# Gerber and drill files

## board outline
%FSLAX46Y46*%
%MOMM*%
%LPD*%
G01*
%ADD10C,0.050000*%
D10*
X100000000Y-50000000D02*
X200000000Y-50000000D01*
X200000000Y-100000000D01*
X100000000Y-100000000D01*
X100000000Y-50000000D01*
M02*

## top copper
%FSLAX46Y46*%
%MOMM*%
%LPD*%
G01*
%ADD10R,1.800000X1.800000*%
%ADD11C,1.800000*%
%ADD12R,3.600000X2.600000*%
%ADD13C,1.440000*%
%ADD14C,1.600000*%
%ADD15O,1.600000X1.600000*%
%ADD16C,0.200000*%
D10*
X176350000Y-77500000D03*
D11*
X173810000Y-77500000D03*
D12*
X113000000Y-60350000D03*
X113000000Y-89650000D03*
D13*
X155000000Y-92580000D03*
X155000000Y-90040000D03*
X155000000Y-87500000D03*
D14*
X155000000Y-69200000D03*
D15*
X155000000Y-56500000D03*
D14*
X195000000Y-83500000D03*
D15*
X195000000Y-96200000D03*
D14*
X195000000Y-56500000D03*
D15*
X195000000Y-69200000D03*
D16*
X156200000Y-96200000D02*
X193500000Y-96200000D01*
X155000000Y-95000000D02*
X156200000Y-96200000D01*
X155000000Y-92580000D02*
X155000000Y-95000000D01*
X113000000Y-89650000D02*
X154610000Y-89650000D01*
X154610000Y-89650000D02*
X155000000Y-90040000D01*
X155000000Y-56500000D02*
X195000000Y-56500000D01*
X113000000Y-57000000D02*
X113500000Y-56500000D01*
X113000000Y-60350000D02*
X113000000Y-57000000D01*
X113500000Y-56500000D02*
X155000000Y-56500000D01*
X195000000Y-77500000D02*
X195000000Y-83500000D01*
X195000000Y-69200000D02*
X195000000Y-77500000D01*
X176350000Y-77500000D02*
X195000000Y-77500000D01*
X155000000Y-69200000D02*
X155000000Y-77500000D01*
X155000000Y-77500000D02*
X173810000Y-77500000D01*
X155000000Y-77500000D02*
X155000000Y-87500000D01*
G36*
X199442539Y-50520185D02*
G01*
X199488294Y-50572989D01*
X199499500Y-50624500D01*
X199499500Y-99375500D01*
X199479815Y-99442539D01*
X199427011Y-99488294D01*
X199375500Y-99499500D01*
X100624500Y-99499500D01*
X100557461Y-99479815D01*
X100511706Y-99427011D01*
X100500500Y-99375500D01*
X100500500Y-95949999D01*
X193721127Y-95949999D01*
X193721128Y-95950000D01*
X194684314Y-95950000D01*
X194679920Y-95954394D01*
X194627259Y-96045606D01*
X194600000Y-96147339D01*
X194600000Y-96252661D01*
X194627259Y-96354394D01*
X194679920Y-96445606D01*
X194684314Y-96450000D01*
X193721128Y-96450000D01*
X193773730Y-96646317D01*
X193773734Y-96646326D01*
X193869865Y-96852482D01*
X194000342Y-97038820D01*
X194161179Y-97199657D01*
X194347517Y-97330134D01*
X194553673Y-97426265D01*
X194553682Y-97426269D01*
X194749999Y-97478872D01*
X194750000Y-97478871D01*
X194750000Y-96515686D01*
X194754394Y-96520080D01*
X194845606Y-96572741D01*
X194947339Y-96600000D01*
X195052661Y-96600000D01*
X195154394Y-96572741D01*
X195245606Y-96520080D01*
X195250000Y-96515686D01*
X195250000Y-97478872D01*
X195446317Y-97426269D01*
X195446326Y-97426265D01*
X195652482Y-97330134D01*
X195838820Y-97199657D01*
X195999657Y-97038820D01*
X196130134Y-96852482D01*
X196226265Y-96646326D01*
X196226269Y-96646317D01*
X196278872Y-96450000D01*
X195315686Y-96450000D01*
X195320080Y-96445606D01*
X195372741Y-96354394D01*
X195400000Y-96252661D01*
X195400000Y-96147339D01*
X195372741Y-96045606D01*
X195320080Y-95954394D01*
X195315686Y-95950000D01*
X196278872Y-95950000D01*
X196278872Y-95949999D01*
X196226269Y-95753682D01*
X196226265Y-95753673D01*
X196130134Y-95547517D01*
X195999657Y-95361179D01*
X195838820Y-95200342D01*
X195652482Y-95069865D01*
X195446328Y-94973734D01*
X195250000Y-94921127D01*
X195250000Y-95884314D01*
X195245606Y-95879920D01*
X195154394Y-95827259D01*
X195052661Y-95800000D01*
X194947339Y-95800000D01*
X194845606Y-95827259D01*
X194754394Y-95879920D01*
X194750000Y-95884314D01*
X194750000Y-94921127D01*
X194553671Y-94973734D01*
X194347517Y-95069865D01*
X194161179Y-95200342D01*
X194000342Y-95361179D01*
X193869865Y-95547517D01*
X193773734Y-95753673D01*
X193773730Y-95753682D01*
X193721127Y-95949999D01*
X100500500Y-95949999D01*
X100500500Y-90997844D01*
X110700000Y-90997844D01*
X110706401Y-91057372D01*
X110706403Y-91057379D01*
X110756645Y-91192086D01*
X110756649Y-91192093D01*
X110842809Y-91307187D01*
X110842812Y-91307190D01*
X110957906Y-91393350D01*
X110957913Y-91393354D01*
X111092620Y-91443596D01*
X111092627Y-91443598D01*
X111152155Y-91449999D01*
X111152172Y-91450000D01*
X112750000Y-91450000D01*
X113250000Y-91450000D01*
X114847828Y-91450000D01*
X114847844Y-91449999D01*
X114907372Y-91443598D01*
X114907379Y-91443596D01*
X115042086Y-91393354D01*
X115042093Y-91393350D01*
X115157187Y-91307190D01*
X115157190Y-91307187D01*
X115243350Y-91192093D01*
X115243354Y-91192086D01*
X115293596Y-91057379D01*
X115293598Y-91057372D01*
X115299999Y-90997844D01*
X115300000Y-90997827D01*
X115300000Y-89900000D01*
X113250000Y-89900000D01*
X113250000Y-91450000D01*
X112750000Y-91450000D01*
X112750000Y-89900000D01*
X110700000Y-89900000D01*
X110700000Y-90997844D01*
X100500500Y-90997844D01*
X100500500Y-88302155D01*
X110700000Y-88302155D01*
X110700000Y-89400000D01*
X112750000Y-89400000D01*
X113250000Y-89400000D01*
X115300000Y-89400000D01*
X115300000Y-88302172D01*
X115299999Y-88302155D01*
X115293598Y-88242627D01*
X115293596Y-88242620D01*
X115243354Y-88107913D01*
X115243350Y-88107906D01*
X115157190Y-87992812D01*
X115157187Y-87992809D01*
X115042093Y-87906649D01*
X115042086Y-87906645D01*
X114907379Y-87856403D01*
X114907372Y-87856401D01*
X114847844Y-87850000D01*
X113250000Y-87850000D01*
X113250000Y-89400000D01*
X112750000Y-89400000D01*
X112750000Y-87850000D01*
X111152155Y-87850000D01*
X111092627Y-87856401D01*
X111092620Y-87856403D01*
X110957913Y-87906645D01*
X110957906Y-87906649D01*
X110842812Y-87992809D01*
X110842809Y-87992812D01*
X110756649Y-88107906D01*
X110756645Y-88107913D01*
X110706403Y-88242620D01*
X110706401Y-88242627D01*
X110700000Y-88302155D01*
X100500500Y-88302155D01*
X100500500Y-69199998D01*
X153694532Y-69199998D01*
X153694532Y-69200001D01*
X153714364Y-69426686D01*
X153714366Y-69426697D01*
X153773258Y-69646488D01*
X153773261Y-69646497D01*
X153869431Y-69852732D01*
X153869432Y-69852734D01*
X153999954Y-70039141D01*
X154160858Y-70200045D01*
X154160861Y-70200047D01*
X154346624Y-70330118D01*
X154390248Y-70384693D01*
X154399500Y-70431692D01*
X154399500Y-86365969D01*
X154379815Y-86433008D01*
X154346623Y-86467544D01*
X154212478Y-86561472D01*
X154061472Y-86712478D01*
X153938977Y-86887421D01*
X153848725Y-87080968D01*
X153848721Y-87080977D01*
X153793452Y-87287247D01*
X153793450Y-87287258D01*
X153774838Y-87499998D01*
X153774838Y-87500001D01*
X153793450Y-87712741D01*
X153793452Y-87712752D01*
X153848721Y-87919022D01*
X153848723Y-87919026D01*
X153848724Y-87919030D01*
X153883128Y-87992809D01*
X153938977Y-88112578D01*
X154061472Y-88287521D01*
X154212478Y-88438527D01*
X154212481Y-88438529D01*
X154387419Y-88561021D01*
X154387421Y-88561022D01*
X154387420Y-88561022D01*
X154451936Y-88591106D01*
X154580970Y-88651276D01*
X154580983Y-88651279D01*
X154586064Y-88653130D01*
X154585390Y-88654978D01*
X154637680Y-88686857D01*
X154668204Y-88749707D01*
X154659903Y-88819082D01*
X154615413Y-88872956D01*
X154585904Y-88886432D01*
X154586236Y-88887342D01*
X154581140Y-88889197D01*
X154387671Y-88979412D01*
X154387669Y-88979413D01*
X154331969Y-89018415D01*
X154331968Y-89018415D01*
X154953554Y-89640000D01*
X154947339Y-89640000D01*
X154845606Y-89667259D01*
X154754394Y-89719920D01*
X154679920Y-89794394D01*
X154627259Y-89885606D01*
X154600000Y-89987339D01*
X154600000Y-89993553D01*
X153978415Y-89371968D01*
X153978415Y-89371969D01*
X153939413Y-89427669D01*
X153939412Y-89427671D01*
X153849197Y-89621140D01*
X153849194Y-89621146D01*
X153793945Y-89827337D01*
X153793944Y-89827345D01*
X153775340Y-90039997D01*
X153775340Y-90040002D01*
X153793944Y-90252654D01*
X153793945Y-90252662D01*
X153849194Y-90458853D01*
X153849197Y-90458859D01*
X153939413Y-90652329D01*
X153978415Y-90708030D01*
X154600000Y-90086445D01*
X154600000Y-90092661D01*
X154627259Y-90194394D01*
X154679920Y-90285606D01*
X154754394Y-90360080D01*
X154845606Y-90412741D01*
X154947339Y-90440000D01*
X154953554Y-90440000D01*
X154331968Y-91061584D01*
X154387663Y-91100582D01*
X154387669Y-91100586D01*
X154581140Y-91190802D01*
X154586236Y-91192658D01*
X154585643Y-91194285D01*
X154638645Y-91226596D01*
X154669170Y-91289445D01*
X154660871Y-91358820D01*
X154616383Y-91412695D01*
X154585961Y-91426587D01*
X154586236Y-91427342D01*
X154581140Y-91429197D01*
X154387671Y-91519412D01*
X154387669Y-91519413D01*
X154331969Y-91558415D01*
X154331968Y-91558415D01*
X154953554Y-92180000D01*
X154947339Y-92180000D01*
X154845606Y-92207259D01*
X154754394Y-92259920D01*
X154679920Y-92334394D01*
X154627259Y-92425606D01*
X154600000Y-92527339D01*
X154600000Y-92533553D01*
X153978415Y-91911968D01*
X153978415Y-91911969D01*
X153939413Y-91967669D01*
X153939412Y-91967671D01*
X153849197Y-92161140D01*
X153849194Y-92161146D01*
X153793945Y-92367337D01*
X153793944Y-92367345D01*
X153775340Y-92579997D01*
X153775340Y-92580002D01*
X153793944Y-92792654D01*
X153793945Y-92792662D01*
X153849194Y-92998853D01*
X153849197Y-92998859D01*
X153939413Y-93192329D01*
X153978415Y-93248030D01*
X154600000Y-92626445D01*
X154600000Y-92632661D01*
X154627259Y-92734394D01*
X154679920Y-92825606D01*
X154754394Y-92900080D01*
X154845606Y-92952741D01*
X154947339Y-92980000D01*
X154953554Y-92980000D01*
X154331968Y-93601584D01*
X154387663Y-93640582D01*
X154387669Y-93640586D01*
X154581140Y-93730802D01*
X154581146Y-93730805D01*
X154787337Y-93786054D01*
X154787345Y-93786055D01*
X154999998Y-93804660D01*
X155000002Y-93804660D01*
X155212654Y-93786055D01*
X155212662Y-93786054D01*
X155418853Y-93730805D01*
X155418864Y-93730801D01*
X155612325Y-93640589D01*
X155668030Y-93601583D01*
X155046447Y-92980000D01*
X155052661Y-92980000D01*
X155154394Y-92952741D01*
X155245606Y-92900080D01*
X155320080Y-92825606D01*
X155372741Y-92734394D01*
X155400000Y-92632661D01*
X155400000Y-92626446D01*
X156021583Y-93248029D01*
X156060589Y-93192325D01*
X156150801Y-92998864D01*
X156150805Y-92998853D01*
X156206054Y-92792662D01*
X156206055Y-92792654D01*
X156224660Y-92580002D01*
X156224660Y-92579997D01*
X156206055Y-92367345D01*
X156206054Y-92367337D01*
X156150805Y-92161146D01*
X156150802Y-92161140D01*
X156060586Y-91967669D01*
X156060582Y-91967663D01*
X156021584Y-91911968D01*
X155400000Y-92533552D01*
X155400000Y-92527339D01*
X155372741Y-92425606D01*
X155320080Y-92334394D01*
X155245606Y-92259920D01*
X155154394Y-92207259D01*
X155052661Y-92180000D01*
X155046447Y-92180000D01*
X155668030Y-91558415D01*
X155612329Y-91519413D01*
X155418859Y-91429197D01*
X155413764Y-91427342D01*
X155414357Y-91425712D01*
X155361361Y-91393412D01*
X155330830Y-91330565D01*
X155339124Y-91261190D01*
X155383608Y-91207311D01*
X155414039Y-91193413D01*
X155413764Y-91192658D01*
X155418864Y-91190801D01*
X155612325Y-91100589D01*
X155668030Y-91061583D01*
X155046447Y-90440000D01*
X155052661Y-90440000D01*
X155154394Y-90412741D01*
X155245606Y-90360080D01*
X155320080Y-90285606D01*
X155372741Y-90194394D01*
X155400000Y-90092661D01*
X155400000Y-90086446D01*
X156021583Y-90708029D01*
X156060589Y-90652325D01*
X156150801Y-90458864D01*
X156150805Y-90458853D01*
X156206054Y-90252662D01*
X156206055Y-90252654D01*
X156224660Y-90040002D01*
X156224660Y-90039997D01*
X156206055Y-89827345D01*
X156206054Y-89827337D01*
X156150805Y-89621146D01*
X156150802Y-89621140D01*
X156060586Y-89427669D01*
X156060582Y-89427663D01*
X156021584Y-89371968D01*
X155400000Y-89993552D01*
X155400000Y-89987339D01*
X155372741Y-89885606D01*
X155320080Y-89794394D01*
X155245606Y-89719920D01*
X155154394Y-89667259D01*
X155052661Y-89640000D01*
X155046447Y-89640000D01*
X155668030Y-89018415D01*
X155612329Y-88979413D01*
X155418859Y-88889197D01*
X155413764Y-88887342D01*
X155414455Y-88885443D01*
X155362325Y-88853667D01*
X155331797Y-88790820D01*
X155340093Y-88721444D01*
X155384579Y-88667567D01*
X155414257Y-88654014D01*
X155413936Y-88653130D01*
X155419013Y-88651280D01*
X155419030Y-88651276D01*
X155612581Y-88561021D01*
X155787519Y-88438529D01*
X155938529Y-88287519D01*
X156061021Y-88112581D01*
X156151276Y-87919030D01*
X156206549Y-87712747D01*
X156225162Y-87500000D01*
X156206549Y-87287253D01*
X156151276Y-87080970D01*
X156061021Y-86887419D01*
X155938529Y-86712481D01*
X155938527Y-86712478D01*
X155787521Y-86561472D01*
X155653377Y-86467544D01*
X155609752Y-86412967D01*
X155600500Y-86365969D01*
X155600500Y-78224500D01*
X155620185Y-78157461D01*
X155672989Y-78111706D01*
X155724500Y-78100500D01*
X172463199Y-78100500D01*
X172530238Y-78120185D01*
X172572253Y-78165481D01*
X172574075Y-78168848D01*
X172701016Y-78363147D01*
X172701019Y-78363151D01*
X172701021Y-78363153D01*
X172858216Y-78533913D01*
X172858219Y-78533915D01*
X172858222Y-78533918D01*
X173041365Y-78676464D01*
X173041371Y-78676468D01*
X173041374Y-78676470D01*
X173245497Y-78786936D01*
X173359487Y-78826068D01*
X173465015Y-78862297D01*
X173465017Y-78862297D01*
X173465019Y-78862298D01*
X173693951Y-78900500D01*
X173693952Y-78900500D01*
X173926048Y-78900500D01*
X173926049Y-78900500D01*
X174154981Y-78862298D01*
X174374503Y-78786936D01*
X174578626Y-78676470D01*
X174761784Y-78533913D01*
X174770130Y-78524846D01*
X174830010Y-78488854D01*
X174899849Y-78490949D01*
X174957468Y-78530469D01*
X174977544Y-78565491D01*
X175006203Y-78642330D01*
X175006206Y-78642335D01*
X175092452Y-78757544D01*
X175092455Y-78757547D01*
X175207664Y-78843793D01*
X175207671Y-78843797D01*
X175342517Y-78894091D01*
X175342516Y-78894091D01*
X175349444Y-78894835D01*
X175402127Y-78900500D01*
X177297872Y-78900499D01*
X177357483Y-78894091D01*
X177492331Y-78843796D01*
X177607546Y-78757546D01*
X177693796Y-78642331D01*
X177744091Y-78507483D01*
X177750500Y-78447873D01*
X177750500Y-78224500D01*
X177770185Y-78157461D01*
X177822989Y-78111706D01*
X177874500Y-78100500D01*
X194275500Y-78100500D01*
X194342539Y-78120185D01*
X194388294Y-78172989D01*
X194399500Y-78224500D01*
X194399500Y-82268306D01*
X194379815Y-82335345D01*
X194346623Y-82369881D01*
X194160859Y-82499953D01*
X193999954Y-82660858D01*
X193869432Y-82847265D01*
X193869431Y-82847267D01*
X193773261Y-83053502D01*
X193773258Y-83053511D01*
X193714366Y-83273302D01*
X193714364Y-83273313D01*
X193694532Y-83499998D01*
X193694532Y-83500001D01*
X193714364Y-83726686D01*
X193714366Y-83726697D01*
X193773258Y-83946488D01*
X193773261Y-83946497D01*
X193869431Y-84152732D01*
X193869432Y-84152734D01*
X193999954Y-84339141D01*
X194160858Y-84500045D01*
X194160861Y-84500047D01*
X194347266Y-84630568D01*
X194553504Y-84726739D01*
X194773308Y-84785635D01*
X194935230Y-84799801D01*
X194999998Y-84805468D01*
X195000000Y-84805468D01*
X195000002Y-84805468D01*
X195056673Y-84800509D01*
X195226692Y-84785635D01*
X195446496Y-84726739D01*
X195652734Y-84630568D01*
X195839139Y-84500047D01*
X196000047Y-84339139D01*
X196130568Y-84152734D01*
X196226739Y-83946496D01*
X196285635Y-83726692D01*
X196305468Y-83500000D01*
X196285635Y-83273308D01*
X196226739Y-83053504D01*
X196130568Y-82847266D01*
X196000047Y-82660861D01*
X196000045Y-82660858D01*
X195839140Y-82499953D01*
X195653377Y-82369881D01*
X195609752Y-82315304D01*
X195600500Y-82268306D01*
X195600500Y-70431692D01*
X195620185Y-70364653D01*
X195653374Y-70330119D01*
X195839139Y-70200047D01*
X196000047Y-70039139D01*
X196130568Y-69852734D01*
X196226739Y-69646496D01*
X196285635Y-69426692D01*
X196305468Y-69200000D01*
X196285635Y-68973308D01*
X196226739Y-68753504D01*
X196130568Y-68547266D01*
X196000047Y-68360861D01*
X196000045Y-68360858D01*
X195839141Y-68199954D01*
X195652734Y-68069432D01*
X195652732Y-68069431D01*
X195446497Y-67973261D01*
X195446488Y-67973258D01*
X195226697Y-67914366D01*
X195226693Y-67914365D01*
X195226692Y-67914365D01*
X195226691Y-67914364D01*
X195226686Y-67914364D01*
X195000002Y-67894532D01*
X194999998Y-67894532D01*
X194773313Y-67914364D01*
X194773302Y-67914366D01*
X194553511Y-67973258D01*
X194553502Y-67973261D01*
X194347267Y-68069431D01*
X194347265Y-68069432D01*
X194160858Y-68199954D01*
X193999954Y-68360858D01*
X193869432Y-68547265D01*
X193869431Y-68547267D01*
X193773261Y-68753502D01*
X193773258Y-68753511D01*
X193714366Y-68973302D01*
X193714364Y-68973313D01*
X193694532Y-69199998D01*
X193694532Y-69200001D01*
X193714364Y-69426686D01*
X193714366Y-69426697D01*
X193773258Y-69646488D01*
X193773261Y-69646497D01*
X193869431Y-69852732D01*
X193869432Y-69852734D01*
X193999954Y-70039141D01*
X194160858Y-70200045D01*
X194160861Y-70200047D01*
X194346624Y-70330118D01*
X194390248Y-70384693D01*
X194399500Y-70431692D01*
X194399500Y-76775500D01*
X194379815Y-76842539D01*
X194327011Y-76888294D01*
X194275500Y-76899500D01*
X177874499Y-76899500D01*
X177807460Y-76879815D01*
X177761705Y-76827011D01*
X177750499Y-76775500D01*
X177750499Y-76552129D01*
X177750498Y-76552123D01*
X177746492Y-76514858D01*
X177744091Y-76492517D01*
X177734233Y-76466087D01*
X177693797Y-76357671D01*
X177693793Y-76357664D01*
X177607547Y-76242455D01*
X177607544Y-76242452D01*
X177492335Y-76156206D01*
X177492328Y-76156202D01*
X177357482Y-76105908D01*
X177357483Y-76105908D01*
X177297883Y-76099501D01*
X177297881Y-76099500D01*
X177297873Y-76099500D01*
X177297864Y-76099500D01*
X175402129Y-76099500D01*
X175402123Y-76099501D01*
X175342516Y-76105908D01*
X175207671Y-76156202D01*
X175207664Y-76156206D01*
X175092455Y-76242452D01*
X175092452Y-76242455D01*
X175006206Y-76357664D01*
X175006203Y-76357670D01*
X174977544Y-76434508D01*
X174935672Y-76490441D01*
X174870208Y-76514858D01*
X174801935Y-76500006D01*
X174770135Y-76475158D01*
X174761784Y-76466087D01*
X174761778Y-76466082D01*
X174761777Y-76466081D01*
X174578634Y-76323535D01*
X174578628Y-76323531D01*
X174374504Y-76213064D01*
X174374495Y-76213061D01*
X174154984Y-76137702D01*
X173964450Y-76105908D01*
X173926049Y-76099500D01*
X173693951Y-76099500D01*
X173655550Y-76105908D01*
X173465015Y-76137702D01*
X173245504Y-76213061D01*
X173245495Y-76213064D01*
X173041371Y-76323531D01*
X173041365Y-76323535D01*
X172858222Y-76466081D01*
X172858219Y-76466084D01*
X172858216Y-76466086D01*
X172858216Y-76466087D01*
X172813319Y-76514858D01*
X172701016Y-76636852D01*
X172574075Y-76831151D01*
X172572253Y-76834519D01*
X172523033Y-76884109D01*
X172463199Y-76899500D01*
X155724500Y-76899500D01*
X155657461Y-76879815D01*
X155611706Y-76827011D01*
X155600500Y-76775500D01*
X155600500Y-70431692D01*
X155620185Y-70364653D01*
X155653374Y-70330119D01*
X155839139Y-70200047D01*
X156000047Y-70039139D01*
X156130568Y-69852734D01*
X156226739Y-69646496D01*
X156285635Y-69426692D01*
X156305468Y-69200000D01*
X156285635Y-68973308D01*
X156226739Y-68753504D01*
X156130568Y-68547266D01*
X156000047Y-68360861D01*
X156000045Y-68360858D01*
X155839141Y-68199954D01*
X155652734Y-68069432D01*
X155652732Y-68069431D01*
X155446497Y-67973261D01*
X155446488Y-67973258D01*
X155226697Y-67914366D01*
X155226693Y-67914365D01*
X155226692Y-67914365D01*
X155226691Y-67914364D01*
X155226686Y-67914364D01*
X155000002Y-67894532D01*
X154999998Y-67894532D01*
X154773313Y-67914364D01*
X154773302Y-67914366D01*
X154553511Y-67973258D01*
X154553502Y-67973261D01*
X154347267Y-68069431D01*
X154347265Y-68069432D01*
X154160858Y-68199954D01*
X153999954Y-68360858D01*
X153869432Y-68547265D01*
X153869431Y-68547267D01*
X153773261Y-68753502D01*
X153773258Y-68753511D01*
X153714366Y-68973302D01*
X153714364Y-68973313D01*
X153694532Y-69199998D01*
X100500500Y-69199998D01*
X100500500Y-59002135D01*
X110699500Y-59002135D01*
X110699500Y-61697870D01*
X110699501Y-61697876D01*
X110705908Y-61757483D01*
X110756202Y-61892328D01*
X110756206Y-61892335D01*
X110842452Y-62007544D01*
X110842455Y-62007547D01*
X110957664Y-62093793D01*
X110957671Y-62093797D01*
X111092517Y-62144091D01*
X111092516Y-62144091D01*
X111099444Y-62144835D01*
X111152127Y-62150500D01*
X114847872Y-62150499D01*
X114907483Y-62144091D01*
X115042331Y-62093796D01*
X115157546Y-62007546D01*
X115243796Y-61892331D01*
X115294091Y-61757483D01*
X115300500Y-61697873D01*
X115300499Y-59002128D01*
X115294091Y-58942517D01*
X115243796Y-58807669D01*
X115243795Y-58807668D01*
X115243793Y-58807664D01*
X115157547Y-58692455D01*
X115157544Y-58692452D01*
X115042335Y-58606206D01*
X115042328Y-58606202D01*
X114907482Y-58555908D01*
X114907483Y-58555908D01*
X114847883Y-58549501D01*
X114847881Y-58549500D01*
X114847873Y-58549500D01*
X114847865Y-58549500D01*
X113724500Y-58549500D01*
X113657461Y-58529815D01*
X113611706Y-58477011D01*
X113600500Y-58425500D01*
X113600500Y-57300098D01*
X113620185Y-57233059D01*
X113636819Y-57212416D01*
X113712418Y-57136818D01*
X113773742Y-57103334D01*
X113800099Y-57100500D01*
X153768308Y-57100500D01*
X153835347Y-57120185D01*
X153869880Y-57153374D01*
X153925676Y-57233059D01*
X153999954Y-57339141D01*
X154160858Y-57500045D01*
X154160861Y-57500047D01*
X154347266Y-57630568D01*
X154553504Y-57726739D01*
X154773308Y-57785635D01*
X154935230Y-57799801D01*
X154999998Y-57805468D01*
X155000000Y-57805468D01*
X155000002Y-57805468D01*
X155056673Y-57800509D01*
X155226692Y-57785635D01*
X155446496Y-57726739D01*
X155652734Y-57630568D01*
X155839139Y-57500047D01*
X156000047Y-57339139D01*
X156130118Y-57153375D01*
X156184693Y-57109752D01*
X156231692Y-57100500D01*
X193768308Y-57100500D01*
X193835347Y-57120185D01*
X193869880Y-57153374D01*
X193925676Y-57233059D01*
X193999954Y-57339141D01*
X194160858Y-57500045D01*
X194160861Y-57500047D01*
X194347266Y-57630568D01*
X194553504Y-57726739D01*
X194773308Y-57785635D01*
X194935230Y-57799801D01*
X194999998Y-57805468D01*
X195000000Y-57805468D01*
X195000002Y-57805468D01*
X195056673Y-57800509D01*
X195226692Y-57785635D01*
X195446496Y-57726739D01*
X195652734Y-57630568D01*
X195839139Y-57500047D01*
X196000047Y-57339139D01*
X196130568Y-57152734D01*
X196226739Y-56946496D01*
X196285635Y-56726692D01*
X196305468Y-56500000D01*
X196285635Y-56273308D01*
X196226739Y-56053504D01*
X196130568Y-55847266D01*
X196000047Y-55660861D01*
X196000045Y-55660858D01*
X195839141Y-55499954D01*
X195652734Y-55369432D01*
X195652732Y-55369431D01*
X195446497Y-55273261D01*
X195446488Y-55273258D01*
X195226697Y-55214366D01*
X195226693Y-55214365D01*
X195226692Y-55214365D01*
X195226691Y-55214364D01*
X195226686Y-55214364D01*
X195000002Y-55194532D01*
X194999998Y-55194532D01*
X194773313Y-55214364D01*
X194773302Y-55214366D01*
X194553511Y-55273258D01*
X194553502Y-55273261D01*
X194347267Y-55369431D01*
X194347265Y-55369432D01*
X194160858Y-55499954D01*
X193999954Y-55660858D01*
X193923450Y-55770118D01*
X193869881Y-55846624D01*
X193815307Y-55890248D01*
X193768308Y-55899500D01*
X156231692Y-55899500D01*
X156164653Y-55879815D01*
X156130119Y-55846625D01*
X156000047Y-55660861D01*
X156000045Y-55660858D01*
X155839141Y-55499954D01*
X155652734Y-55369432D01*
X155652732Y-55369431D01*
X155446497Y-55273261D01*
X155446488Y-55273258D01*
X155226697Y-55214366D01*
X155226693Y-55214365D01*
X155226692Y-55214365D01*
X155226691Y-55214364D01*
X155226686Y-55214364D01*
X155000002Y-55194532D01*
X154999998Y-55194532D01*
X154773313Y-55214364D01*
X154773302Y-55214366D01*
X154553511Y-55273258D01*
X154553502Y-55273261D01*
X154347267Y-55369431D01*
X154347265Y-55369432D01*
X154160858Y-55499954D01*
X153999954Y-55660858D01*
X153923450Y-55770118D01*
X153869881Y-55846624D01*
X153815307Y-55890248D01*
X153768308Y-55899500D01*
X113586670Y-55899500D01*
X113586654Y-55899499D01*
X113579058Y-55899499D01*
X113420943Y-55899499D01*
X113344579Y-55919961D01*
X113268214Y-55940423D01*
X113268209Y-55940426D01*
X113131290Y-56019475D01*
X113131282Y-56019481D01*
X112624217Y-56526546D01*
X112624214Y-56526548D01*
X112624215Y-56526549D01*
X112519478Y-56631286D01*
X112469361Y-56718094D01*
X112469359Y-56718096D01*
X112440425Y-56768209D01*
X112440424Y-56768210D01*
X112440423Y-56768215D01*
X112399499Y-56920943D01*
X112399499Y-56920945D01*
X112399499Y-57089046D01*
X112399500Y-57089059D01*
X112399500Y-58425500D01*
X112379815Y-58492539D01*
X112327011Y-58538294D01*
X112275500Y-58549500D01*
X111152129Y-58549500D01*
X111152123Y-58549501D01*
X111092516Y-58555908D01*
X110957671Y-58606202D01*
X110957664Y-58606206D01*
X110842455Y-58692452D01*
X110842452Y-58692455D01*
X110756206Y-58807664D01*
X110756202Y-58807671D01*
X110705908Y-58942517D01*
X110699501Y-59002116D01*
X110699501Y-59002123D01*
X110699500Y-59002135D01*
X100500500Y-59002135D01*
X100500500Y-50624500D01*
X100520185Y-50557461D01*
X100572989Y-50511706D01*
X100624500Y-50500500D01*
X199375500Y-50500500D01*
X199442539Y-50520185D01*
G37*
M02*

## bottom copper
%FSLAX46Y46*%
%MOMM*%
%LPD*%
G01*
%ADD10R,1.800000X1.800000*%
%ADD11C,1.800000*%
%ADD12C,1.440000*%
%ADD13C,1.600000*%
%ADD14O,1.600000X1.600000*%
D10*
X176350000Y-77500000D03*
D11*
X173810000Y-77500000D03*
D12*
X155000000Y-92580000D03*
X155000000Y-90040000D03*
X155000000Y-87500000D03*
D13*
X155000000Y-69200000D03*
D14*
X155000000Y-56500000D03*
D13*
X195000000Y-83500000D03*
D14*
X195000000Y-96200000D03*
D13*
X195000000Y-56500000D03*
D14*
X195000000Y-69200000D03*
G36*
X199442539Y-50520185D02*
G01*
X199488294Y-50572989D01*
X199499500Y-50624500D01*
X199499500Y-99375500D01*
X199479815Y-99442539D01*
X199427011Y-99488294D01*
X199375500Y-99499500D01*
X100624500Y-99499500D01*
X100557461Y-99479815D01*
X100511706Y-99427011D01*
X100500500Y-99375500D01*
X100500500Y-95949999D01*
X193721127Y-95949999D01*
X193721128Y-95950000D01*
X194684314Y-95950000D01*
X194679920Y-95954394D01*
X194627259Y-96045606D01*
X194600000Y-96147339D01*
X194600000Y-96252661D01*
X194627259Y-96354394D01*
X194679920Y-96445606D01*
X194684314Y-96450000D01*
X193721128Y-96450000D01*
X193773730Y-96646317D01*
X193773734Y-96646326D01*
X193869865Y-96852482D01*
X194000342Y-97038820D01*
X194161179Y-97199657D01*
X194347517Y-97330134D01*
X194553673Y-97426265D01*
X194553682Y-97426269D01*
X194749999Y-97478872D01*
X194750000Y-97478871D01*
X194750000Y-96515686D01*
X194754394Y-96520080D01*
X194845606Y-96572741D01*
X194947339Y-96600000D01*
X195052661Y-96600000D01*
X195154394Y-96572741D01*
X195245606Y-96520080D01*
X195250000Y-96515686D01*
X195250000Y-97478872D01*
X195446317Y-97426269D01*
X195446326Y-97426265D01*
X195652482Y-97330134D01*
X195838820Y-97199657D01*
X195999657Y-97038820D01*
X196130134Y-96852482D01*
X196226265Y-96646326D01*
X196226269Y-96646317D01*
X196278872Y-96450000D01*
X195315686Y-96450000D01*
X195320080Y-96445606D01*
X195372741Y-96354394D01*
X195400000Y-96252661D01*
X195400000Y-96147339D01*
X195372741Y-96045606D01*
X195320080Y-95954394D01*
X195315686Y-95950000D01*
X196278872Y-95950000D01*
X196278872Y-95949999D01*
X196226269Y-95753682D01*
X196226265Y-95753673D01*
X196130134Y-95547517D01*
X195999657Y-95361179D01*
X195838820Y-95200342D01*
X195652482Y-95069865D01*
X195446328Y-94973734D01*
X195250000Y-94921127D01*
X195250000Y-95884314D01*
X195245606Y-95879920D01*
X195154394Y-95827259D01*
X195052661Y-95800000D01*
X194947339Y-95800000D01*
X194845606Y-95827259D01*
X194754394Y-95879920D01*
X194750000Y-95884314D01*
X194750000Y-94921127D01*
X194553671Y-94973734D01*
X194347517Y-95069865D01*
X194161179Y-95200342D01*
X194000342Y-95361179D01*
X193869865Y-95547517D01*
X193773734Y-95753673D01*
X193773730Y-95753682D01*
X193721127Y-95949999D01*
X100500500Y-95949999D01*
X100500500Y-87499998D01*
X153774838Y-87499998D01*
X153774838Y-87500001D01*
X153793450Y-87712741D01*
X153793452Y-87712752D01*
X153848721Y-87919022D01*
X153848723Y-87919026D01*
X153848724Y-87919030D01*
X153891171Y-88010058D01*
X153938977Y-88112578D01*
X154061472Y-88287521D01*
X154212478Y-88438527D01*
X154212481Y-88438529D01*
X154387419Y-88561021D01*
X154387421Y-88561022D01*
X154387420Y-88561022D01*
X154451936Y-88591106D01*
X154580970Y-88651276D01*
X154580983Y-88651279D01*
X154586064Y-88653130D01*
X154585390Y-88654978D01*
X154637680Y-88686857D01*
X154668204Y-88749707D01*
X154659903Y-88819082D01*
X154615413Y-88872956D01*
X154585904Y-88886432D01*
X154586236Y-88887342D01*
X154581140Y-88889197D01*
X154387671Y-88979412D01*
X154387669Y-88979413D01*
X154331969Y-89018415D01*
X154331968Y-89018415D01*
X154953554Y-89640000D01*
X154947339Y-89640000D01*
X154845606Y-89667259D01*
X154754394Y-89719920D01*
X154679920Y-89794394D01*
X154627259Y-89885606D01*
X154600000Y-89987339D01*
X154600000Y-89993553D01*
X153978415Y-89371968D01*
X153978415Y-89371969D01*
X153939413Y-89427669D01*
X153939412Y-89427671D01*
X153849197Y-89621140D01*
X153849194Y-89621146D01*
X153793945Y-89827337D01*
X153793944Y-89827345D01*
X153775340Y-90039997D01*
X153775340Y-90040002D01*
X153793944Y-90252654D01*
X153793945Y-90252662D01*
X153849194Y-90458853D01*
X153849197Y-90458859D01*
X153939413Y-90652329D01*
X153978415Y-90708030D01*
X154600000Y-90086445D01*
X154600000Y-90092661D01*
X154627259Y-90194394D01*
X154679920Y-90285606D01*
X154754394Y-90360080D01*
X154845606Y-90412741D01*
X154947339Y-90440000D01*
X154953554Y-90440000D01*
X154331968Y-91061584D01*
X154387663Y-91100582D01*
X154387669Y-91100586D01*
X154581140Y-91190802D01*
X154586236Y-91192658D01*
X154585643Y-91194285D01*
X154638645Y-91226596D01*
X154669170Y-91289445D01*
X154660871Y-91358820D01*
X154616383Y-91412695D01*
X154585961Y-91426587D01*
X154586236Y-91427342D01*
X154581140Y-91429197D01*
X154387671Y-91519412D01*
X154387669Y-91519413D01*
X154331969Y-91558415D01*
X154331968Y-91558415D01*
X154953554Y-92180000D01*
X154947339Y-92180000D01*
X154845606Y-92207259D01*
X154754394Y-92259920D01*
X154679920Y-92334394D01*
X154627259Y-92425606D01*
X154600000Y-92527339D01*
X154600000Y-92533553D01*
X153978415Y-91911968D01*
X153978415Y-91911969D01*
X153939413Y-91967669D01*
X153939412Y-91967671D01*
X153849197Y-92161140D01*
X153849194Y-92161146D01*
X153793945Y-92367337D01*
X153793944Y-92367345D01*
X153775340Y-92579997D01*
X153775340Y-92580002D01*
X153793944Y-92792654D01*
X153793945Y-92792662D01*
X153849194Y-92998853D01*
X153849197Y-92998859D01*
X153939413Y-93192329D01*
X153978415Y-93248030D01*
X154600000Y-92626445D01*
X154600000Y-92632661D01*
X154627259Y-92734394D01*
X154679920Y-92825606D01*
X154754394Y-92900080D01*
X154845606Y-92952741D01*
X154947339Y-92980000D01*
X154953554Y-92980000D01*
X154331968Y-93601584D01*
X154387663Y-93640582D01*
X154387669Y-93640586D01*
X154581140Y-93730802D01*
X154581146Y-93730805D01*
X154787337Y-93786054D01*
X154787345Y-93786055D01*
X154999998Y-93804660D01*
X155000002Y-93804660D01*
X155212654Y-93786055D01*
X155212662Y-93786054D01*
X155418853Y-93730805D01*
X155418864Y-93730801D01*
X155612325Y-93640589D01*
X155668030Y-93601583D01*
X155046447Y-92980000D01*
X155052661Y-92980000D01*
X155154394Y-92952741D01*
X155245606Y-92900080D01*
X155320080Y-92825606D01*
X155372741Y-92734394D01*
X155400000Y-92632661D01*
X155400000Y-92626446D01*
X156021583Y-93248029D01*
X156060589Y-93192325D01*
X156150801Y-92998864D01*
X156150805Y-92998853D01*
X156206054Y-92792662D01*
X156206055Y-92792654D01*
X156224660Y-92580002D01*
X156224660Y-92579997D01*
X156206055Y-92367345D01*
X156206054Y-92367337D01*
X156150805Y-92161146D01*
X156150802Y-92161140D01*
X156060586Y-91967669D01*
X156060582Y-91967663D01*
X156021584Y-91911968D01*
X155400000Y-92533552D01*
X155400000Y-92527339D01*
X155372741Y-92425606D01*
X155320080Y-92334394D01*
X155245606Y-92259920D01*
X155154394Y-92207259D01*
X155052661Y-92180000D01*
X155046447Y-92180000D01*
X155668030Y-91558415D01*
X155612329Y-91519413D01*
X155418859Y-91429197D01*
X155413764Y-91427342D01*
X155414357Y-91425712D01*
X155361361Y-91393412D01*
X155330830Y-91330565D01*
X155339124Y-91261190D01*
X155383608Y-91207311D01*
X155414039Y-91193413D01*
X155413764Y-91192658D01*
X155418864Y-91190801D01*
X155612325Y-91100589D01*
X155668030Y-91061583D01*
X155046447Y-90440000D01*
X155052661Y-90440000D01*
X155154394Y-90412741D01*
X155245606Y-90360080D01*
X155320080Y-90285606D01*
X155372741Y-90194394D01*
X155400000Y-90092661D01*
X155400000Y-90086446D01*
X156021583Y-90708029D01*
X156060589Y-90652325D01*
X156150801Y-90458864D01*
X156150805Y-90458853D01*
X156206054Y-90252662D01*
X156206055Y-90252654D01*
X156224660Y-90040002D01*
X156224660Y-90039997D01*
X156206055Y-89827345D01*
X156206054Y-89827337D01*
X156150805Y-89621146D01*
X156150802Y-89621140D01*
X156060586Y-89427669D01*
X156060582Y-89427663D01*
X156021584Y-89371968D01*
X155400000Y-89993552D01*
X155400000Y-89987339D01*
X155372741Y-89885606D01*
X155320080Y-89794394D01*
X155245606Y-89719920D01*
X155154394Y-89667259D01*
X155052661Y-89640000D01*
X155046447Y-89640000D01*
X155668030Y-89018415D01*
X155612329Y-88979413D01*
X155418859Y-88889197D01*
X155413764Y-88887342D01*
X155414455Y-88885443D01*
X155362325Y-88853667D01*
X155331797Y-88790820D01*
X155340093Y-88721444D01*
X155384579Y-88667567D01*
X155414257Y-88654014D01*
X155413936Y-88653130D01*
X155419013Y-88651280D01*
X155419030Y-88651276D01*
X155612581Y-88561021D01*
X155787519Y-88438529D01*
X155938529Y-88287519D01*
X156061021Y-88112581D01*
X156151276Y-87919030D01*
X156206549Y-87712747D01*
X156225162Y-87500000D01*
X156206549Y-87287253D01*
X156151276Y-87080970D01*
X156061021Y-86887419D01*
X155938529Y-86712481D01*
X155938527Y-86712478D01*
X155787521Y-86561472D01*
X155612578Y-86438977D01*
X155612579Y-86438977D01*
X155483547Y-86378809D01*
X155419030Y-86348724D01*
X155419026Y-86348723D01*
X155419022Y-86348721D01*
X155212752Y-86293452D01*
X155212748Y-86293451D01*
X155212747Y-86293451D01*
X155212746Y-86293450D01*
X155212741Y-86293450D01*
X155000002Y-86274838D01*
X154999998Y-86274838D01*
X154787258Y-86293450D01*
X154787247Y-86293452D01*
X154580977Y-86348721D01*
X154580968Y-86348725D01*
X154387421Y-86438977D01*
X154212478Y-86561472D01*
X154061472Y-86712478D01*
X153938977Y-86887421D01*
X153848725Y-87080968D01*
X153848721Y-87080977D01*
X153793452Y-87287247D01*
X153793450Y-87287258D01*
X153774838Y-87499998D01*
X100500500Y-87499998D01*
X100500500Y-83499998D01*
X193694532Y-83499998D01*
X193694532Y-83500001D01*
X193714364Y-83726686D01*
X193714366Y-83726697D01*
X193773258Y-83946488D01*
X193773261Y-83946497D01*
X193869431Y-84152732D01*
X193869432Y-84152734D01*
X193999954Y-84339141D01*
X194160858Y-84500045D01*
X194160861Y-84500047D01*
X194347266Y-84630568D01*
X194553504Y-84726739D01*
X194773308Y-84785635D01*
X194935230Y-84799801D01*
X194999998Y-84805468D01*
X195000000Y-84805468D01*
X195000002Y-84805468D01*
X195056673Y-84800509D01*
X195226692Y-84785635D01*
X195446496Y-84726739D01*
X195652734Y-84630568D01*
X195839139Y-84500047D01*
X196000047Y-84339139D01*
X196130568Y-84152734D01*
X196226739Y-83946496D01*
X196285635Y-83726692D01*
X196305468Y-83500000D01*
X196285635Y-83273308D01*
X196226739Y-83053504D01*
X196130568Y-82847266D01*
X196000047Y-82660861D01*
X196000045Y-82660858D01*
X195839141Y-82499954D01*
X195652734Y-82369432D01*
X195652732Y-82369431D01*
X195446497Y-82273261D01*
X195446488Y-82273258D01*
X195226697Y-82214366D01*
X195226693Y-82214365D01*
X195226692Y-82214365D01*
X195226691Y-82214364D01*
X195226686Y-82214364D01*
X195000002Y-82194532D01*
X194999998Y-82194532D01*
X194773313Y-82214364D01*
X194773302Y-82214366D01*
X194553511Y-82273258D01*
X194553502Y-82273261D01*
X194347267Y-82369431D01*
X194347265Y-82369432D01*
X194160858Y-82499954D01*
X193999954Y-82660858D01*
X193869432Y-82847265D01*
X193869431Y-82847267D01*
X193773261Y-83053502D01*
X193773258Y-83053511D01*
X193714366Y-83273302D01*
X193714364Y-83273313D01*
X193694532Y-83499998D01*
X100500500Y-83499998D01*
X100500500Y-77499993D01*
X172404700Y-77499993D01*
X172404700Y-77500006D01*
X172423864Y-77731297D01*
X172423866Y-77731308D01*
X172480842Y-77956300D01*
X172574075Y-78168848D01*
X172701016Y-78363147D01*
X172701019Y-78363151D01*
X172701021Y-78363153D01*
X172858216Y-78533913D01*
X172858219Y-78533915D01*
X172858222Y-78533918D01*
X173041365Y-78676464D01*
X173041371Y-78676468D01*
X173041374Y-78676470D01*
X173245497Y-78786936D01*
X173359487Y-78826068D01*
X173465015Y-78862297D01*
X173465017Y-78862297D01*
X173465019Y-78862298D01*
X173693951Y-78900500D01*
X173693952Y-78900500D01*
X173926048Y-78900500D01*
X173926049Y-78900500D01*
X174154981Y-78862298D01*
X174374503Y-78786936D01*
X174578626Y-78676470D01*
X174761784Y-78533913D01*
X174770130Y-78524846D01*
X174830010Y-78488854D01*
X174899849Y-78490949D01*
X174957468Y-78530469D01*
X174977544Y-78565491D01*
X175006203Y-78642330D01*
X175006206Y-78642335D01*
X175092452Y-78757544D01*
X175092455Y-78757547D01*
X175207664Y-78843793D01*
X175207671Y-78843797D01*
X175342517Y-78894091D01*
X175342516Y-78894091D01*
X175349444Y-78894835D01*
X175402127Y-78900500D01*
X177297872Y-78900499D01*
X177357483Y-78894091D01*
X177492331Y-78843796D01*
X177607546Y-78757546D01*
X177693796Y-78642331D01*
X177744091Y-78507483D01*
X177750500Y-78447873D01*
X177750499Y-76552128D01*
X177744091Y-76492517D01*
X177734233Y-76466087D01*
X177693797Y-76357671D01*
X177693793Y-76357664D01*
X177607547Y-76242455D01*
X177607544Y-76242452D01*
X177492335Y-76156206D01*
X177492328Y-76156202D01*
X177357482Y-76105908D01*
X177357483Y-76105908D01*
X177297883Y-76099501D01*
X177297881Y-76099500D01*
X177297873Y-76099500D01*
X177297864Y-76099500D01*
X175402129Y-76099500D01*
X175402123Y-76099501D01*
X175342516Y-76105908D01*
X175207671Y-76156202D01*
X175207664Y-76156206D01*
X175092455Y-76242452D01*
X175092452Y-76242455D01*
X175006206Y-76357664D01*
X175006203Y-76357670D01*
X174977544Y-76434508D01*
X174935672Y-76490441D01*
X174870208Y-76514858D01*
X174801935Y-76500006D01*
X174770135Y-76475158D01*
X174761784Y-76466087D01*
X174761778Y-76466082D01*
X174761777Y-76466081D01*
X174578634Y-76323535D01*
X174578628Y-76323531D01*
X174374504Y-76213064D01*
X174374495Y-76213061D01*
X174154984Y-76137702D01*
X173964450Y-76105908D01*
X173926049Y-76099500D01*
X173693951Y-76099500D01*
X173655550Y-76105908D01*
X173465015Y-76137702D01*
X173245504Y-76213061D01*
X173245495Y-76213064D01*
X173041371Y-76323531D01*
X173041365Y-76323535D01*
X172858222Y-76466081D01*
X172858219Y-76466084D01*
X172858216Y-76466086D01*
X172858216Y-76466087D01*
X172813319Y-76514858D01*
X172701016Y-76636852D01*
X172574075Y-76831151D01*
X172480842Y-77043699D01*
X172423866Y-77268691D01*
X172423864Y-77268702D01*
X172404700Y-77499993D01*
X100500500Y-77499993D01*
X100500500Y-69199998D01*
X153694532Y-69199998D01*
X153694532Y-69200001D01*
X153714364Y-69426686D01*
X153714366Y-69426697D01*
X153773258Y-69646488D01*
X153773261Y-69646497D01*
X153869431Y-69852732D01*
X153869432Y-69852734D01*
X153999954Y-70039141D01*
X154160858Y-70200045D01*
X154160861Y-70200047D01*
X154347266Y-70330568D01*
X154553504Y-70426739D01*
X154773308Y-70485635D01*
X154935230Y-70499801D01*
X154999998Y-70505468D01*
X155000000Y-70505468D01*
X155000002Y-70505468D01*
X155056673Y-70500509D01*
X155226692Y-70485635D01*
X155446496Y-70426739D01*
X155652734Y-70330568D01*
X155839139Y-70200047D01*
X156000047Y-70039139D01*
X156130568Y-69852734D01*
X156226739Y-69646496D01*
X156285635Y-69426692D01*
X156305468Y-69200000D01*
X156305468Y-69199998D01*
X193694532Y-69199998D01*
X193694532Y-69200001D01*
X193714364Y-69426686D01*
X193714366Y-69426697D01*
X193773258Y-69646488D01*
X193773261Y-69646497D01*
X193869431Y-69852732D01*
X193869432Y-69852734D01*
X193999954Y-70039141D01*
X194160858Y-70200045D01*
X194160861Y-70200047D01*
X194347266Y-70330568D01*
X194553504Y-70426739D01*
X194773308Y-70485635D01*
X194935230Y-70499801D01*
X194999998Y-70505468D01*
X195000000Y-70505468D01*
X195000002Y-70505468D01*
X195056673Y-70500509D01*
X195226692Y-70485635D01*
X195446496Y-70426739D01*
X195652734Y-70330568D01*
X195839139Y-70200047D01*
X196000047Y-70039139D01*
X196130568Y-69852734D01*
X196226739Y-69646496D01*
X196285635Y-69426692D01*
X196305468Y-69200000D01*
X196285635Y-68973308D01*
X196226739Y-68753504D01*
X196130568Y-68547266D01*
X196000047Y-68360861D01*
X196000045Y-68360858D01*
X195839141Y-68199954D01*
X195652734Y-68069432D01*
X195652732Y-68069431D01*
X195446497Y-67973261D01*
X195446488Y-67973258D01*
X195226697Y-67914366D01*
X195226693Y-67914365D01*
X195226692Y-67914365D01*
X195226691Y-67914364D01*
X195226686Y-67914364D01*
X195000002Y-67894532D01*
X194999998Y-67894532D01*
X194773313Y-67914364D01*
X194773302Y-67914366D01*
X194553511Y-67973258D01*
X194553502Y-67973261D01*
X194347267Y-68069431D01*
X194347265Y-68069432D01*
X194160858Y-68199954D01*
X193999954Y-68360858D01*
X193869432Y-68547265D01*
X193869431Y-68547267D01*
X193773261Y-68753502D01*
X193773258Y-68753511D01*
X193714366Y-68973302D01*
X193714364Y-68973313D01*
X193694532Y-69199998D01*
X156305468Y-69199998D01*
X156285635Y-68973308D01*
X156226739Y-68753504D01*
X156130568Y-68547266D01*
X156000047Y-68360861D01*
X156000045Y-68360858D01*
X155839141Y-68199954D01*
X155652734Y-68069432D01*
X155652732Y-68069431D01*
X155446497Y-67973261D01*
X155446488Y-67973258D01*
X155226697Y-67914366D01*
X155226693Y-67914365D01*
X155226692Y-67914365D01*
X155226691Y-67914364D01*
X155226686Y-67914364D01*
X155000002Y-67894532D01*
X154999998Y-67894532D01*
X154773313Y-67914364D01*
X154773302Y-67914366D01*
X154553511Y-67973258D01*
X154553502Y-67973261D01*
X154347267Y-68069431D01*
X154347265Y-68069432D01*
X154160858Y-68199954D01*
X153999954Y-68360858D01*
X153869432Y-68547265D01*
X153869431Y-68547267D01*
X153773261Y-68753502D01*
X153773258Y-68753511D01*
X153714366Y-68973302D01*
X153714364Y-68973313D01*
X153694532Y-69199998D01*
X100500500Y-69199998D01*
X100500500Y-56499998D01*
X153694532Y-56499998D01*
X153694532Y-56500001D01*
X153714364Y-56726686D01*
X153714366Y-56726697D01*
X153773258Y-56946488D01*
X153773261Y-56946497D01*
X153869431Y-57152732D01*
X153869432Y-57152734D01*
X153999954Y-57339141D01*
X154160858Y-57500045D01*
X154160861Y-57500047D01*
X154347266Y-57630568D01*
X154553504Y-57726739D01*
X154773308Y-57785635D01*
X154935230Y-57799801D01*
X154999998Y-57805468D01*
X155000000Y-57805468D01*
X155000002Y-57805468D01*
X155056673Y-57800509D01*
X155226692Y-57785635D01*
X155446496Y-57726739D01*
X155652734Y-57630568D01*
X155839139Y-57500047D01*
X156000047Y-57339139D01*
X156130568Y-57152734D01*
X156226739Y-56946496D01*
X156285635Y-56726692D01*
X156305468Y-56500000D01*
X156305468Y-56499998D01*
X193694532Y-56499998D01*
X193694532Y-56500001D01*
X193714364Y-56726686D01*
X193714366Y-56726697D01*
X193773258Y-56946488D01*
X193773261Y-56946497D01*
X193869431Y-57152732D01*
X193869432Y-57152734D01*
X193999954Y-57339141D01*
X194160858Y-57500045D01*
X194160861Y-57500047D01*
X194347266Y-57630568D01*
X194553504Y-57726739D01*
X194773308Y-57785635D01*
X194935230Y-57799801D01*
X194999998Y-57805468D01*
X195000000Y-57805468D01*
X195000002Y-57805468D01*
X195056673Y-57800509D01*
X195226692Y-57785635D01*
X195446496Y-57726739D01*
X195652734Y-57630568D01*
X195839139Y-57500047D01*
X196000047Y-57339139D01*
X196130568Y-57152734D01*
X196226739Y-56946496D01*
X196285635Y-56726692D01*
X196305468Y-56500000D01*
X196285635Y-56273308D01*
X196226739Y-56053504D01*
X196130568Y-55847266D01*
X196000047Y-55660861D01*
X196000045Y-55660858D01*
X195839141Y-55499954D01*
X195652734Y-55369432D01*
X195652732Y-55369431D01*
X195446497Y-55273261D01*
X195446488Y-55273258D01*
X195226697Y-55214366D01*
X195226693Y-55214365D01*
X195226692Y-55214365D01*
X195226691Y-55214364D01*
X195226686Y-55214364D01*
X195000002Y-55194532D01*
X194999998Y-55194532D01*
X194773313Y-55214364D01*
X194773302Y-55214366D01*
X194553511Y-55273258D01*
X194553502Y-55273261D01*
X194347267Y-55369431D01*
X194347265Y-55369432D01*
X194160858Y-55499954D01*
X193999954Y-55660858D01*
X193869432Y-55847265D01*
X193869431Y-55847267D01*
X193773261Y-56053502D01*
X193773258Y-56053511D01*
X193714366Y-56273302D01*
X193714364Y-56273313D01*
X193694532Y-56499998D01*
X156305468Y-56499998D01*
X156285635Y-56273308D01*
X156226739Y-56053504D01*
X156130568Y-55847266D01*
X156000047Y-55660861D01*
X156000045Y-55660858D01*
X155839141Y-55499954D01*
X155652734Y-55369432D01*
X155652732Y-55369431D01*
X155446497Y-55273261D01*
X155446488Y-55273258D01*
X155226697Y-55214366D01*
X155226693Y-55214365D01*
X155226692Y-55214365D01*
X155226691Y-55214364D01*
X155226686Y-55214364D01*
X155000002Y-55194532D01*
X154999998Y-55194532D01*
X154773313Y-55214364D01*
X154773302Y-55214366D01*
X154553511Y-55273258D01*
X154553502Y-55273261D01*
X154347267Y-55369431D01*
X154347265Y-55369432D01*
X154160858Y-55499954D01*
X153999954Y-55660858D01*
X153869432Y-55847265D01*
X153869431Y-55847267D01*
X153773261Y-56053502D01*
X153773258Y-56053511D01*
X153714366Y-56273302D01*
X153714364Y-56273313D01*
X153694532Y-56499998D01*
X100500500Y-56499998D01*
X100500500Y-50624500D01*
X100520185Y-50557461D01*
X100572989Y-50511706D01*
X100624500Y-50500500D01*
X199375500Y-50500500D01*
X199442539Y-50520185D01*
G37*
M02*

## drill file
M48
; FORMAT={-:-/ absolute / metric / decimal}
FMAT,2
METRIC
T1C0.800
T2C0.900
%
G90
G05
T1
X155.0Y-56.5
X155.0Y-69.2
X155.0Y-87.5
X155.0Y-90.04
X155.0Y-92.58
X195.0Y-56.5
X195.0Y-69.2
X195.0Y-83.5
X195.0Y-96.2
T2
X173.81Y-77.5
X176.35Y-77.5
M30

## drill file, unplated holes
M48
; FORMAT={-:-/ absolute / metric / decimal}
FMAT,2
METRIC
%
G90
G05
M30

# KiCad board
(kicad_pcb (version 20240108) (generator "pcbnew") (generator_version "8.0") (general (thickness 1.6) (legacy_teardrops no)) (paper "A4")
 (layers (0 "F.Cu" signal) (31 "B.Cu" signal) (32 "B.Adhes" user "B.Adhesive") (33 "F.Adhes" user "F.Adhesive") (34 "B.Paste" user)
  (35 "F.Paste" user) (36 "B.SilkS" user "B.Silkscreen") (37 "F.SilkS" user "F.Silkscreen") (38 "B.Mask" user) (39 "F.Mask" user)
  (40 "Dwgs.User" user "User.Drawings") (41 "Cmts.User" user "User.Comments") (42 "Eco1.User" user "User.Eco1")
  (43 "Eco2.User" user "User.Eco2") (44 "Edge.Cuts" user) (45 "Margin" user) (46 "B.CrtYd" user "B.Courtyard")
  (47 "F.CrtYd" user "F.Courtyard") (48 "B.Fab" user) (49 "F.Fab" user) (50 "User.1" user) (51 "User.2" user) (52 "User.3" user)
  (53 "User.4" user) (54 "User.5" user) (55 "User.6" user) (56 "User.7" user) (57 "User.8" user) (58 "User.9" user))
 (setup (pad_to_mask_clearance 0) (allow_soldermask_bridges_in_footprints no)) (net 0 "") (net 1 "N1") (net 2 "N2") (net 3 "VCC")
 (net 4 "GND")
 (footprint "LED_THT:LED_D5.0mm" (layer "F.Cu") (at 176.35 77.5 180)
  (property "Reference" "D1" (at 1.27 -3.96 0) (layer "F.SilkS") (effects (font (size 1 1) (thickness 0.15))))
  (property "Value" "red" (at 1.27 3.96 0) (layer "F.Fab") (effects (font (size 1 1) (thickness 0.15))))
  (pad "1" thru_hole rect (at 0 0 180) (size 1.8 1.8) (drill 0.9) (layers "*.Cu" "*.Mask") (remove_unused_layers no) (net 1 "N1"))
  (pad "2" thru_hole circle (at 2.54 0 180) (size 1.8 1.8) (drill 0.9) (layers "*.Cu" "*.Mask") (remove_unused_layers no) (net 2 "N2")))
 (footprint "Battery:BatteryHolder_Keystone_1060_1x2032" (layer "F.Cu") (at 113 75 -90)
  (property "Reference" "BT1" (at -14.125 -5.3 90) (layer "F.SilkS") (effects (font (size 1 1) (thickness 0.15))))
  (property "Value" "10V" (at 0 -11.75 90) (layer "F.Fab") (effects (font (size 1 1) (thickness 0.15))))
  (pad "1" smd rect (at -14.65 0 90) (size 2.6 3.6) (layers "F.Cu" "F.Paste" "F.Mask") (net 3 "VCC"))
  (pad "2" smd rect (at 14.65 0 90) (size 2.6 3.6) (layers "F.Cu" "F.Paste" "F.Mask") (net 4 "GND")))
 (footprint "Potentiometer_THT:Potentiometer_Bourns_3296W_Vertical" (layer "F.Cu") (at 155 92.58 -90)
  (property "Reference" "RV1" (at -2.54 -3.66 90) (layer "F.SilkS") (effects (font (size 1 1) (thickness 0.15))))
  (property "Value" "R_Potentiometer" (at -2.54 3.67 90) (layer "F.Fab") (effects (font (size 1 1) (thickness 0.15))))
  (pad "1" thru_hole circle (at 0 0 270) (size 1.44 1.44) (drill 0.8) (layers "*.Cu" "*.Mask") (remove_unused_layers no) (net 4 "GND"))
  (pad "2" thru_hole circle (at -2.54 0 270) (size 1.44 1.44) (drill 0.8) (layers "*.Cu" "*.Mask") (remove_unused_layers no) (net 4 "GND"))
  (pad "3" thru_hole circle (at -5.08 0 270) (size 1.44 1.44) (drill 0.8) (layers "*.Cu" "*.Mask") (remove_unused_layers no) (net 2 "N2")))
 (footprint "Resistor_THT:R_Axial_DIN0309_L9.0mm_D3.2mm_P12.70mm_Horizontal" (layer "F.Cu") (at 155 69.2 90)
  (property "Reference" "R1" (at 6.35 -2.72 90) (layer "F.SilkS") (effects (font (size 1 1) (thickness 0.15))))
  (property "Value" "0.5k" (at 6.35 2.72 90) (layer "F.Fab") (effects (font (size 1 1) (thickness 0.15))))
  (pad "1" thru_hole circle (at 0 0 90) (size 1.6 1.6) (drill 0.8) (layers "*.Cu" "*.Mask") (remove_unused_layers no) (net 2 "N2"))
  (pad "2" thru_hole oval (at 12.7 0 90) (size 1.6 1.6) (drill 0.8) (layers "*.Cu" "*.Mask") (remove_unused_layers no) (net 3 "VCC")))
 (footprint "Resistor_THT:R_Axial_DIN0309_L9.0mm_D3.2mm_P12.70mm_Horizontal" (layer "F.Cu") (at 195 83.5 -90)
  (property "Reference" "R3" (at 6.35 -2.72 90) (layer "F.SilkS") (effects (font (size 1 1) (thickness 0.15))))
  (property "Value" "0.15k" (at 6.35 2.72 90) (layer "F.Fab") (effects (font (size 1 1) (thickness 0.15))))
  (pad "1" thru_hole circle (at 0 0 270) (size 1.6 1.6) (drill 0.8) (layers "*.Cu" "*.Mask") (remove_unused_layers no) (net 1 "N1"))
  (pad "2" thru_hole oval (at 12.7 0 270) (size 1.6 1.6) (drill 0.8) (layers "*.Cu" "*.Mask") (remove_unused_layers no) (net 4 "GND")))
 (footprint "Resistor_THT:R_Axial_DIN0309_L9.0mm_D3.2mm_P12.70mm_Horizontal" (layer "F.Cu") (at 195 56.5 -90)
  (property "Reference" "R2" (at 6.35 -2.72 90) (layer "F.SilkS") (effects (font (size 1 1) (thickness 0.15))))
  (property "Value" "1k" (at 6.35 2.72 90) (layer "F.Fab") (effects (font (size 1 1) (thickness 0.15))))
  (pad "1" thru_hole circle (at 0 0 270) (size 1.6 1.6) (drill 0.8) (layers "*.Cu" "*.Mask") (remove_unused_layers no) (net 3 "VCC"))
  (pad "2" thru_hole oval (at 12.7 0 270) (size 1.6 1.6) (drill 0.8) (layers "*.Cu" "*.Mask") (remove_unused_layers no) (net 1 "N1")))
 (gr_rect (start 100 50) (end 200 100) (stroke (width 0.05) (type default)) (fill none) (layer "Edge.Cuts"))
 (segment (start 156.2 96.2) (end 193.5 96.2) (width 0.2) (layer "F.Cu") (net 4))
 (segment (start 155 95) (end 156.2 96.2) (width 0.2) (layer "F.Cu") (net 4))
 (segment (start 155 92.58) (end 155 95) (width 0.2) (layer "F.Cu") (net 4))
 (segment (start 113 89.65) (end 154.61 89.65) (width 0.2) (layer "F.Cu") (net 4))
 (segment (start 154.61 89.65) (end 155 90.04) (width 0.2) (layer "F.Cu") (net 4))
 (segment (start 155 56.5) (end 195 56.5) (width 0.2) (layer "F.Cu") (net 3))
 (segment (start 113 57) (end 113.5 56.5) (width 0.2) (layer "F.Cu") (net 3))
 (segment (start 113 60.35) (end 113 57) (width 0.2) (layer "F.Cu") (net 3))
 (segment (start 113.5 56.5) (end 155 56.5) (width 0.2) (layer "F.Cu") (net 3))
 (segment (start 195 77.5) (end 195 83.5) (width 0.2) (layer "F.Cu") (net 1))
 (segment (start 195 69.2) (end 195 77.5) (width 0.2) (layer "F.Cu") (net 1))
 (segment (start 176.35 77.5) (end 195 77.5) (width 0.2) (layer "F.Cu") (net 1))
 (segment (start 155 69.2) (end 155 77.5) (width 0.2) (layer "F.Cu") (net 2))
 (segment (start 155 77.5) (end 173.81 77.5) (width 0.2) (layer "F.Cu") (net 2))
 (segment (start 155 77.5) (end 155 87.5) (width 0.2) (layer "F.Cu") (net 2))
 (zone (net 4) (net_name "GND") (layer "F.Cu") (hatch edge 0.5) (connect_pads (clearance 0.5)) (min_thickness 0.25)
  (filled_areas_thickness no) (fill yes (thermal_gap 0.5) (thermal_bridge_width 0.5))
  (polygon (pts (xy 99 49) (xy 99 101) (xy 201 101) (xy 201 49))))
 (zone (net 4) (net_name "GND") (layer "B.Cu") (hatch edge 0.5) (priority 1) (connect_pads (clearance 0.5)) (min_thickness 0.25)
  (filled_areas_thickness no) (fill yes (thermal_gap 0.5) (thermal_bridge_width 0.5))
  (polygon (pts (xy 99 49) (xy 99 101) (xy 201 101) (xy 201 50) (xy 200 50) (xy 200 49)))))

